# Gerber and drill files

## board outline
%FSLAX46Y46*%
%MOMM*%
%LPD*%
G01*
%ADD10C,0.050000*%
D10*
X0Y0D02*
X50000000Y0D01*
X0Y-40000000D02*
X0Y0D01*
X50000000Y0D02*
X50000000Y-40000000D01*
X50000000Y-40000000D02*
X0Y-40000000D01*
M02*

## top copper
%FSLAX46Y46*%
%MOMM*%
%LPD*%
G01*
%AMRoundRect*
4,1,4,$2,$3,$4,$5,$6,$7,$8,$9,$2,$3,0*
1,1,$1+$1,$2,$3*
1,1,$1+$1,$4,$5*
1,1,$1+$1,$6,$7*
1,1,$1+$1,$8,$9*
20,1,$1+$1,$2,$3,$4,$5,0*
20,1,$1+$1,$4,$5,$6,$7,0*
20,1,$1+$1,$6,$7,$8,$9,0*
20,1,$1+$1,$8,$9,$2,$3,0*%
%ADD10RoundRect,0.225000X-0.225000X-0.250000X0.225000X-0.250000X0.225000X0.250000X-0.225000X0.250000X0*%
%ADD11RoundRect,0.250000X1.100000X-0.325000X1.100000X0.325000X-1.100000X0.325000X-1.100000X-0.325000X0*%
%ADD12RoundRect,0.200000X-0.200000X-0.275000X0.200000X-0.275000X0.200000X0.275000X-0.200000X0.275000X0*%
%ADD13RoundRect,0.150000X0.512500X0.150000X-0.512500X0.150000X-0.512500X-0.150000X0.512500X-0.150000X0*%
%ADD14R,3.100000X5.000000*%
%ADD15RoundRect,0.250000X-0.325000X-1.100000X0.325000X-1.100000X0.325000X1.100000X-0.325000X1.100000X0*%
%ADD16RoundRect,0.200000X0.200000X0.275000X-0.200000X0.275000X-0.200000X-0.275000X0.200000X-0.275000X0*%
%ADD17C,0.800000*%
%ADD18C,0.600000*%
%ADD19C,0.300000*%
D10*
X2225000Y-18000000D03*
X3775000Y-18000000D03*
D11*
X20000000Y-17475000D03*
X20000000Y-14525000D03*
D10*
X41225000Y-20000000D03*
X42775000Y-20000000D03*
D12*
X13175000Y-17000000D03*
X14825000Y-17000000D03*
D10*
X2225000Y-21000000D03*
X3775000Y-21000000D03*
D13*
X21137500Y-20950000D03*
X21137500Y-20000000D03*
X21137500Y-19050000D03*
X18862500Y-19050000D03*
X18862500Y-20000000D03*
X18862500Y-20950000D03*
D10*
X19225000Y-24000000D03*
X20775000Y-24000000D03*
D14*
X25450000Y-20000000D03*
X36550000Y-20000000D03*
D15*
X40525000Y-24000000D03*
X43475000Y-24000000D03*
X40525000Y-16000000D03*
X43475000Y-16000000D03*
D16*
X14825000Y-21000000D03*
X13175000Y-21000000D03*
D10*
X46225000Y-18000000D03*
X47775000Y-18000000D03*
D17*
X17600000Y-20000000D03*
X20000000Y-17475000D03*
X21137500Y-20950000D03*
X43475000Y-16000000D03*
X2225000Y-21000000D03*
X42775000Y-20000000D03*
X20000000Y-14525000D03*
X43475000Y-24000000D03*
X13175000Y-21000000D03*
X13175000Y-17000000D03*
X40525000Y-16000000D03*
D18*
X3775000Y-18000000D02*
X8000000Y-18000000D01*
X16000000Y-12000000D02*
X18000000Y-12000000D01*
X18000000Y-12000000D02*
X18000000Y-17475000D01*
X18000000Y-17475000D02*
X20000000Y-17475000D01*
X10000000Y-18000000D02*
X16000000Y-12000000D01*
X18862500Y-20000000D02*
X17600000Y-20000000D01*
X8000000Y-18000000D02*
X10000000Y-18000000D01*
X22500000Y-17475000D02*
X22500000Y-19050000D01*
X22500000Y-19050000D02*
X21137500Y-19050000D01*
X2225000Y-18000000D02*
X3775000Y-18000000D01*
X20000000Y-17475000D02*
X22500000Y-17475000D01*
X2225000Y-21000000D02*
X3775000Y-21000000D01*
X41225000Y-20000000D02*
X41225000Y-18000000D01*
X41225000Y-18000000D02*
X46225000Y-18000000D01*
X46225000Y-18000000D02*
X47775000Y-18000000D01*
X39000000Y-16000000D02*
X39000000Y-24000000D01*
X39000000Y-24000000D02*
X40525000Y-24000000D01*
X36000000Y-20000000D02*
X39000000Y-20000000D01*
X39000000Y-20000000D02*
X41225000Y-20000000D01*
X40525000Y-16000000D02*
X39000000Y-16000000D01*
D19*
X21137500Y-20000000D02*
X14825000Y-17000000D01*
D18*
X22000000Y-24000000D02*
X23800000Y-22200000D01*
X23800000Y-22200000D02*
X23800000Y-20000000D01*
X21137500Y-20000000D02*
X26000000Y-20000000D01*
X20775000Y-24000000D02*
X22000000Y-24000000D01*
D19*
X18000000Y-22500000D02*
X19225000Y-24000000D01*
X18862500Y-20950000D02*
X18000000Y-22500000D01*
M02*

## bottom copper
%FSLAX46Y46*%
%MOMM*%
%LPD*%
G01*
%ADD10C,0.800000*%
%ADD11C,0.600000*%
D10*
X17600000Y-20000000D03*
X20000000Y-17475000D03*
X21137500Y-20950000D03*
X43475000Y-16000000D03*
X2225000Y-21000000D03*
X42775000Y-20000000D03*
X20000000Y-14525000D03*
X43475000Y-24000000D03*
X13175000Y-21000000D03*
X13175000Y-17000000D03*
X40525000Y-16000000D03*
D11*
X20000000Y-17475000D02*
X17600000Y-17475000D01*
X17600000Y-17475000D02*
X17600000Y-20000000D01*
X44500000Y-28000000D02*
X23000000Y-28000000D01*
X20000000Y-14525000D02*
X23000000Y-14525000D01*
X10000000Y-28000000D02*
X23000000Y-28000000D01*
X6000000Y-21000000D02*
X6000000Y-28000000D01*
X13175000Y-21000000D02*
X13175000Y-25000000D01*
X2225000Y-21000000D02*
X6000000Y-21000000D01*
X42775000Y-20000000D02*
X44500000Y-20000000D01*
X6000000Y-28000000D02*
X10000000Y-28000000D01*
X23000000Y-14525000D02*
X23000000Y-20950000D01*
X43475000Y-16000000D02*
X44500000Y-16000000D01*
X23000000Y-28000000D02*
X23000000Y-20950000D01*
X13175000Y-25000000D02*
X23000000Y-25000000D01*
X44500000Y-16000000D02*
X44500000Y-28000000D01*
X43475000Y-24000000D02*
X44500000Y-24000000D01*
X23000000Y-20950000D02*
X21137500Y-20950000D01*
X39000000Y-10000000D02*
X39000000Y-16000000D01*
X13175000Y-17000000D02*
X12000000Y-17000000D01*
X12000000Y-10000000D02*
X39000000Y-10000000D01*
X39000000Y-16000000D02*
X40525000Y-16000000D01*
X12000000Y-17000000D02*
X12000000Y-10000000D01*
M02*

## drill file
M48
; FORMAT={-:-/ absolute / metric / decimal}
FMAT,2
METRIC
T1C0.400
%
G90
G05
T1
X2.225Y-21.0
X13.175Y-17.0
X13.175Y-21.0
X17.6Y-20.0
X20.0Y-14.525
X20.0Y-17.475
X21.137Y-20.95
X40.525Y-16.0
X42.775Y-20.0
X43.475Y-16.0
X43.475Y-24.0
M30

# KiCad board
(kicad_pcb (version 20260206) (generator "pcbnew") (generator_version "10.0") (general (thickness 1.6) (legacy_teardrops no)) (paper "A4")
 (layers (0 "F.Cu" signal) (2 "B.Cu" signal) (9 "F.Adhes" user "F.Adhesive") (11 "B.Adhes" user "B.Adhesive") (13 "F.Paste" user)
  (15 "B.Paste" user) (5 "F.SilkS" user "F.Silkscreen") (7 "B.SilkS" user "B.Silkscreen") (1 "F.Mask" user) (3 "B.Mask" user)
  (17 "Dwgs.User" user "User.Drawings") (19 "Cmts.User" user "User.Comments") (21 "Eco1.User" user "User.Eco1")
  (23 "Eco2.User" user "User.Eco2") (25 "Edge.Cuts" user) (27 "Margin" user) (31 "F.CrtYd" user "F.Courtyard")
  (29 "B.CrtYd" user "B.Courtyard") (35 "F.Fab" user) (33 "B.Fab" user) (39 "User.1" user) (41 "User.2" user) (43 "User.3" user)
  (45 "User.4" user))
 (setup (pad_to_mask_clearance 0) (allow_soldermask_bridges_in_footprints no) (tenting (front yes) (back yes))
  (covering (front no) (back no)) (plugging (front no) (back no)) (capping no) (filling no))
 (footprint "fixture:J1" (layer "F.Cu") (at 3 18)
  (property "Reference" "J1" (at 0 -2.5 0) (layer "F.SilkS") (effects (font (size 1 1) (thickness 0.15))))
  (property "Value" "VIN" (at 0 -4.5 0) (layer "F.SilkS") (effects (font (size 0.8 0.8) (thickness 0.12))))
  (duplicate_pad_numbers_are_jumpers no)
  (pad "1" smd roundrect (at -0.775 0) (size 0.9 0.95) (layers "F.Cu" "F.Mask" "F.Paste") (roundrect_rratio 0.25) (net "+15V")
   (thermal_bridge_angle 45))
  (pad "2" smd roundrect (at 0.775 0) (size 0.9 0.95) (layers "F.Cu" "F.Mask" "F.Paste") (roundrect_rratio 0.25) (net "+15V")
   (thermal_bridge_angle 45)))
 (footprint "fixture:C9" (layer "F.Cu") (at 20 16 90)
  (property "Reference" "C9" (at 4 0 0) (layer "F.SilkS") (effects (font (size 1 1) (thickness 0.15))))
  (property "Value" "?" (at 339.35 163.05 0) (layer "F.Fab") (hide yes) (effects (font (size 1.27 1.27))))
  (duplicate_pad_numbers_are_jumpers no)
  (pad "1" smd roundrect (at -1.475 0 90) (size 1.15 2.7) (layers "F.Cu" "F.Mask" "F.Paste") (roundrect_rratio 0.217391) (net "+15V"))
  (pad "2" smd roundrect (at 1.475 0 90) (size 1.15 2.7) (layers "F.Cu" "F.Mask" "F.Paste") (roundrect_rratio 0.217391) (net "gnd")))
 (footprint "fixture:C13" (layer "F.Cu") (at 42 20)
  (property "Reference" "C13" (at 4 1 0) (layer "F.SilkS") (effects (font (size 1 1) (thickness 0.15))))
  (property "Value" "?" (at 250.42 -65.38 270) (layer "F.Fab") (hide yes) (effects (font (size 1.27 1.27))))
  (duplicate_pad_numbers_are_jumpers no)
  (pad "1" smd roundrect (at -0.775 0) (size 0.9 0.95) (layers "F.Cu" "F.Mask" "F.Paste") (roundrect_rratio 0.25) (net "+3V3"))
  (pad "2" smd roundrect (at 0.775 0) (size 0.9 0.95) (layers "F.Cu" "F.Mask" "F.Paste") (roundrect_rratio 0.25) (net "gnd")))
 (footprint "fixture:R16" (layer "F.Cu") (at 14 17)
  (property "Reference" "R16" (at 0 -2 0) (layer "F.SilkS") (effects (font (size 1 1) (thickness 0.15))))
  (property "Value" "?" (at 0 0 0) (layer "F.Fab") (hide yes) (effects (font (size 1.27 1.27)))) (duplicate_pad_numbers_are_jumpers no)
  (pad "1" smd roundrect (at -0.825 0) (size 0.8 0.95) (layers "F.Cu" "F.Mask" "F.Paste") (roundrect_rratio 0.25) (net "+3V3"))
  (pad "2" smd roundrect (at 0.825 0) (size 0.8 0.95) (layers "F.Cu" "F.Mask" "F.Paste") (roundrect_rratio 0.25) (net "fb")))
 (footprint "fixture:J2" (layer "F.Cu") (at 3 21)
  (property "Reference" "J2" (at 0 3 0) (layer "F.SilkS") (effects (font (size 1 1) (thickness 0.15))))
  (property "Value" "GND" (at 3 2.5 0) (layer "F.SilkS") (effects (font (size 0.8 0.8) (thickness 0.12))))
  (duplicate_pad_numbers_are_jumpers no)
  (pad "1" smd roundrect (at -0.775 0) (size 0.9 0.95) (layers "F.Cu" "F.Mask" "F.Paste") (roundrect_rratio 0.25) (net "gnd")
   (thermal_bridge_angle 45))
  (pad "2" smd roundrect (at 0.775 0) (size 0.9 0.95) (layers "F.Cu" "F.Mask" "F.Paste") (roundrect_rratio 0.25) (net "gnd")
   (thermal_bridge_angle 45)))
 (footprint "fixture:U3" (layer "F.Cu") (at 20 20 180)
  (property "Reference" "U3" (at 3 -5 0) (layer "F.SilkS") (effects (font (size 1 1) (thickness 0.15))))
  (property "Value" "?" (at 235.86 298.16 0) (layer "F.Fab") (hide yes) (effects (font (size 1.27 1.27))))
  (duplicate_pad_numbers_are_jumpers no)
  (pad "1" smd roundrect (at -1.1375 -0.95 180) (size 1.325 0.6) (layers "F.Cu" "F.Mask" "F.Paste") (roundrect_rratio 0.25) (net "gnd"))
  (pad "2" smd roundrect (at -1.1375 0 180) (size 1.325 0.6) (layers "F.Cu" "F.Mask" "F.Paste") (roundrect_rratio 0.25) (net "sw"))
  (pad "3" smd roundrect (at -1.1375 0.95 180) (size 1.325 0.6) (layers "F.Cu" "F.Mask" "F.Paste") (roundrect_rratio 0.25) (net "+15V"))
  (pad "4" smd roundrect (at 1.1375 0.95 180) (size 1.325 0.6) (layers "F.Cu" "F.Mask" "F.Paste") (roundrect_rratio 0.25) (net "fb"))
  (pad "5" smd roundrect (at 1.1375 0 180) (size 1.325 0.6) (layers "F.Cu" "F.Mask" "F.Paste") (roundrect_rratio 0.25) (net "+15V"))
  (pad "6" smd roundrect (at 1.1375 -0.95 180) (size 1.325 0.6) (layers "F.Cu" "F.Mask" "F.Paste") (roundrect_rratio 0.25) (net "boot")))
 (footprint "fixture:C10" (layer "F.Cu") (at 20 24)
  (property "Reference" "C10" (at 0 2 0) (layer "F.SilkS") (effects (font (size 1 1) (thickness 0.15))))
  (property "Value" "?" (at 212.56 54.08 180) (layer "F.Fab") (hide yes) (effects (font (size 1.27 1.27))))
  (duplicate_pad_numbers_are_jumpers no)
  (pad "1" smd roundrect (at -0.775 0) (size 0.9 0.95) (layers "F.Cu" "F.Mask" "F.Paste") (roundrect_rratio 0.25) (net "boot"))
  (pad "2" smd roundrect (at 0.775 0) (size 0.9 0.95) (layers "F.Cu" "F.Mask" "F.Paste") (roundrect_rratio 0.25) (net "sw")))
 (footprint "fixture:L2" (layer "F.Cu") (at 31 20)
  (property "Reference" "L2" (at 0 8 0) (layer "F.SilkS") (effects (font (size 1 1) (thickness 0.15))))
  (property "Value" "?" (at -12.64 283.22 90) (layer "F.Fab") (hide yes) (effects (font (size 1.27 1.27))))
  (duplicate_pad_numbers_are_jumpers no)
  (pad "1" smd rect (at -5.55 0) (size 3.1 5) (layers "F.Cu" "F.Mask" "F.Paste") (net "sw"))
  (pad "2" smd rect (at 5.55 0) (size 3.1 5) (layers "F.Cu" "F.Mask" "F.Paste") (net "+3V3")))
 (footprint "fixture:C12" (layer "F.Cu") (at 42 24)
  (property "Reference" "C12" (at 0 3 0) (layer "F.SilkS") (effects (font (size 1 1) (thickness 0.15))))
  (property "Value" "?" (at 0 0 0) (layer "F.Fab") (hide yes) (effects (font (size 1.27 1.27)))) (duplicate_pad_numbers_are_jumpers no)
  (pad "1" smd roundrect (at -1.475 0) (size 1.15 2.7) (layers "F.Cu" "F.Mask" "F.Paste") (roundrect_rratio 0.217391) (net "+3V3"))
  (pad "2" smd roundrect (at 1.475 0) (size 1.15 2.7) (layers "F.Cu" "F.Mask" "F.Paste") (roundrect_rratio 0.217391) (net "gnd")))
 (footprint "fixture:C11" (layer "F.Cu") (at 42 16)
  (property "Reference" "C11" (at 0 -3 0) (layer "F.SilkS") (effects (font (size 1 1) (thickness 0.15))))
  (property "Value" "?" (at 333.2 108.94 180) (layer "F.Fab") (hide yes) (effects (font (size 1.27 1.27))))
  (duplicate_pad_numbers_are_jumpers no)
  (pad "1" smd roundrect (at -1.475 0) (size 1.15 2.7) (layers "F.Cu" "F.Mask" "F.Paste") (roundrect_rratio 0.217391) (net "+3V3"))
  (pad "2" smd roundrect (at 1.475 0) (size 1.15 2.7) (layers "F.Cu" "F.Mask" "F.Paste") (roundrect_rratio 0.217391) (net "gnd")))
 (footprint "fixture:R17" (layer "F.Cu") (at 14 21 180)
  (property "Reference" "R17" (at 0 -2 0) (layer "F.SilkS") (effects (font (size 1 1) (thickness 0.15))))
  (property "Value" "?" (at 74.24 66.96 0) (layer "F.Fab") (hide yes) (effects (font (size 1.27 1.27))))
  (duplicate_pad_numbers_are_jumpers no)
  (pad "1" smd roundrect (at -0.825 0 180) (size 0.8 0.95) (layers "F.Cu" "F.Mask" "F.Paste") (roundrect_rratio 0.25) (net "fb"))
  (pad "2" smd roundrect (at 0.825 0 180) (size 0.8 0.95) (layers "F.Cu" "F.Mask" "F.Paste") (roundrect_rratio 0.25) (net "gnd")))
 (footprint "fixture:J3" (layer "F.Cu") (at 47 18)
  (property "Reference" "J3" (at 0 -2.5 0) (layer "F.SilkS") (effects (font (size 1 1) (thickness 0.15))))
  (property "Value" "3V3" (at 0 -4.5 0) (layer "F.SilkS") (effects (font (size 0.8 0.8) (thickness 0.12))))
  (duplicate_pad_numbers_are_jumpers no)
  (pad "1" smd roundrect (at -0.775 0) (size 0.9 0.95) (layers "F.Cu" "F.Mask" "F.Paste") (roundrect_rratio 0.25) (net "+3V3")
   (thermal_bridge_angle 45))
  (pad "2" smd roundrect (at 0.775 0) (size 0.9 0.95) (layers "F.Cu" "F.Mask" "F.Paste") (roundrect_rratio 0.25) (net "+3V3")
   (thermal_bridge_angle 45)))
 (gr_line (start 0 0) (end 50 0) (stroke (width 0.05) (type default)) (layer "Edge.Cuts"))
 (gr_line (start 0 40) (end 0 0) (stroke (width 0.05) (type default)) (layer "Edge.Cuts"))
 (gr_line (start 50 0) (end 50 40) (stroke (width 0.05) (type default)) (layer "Edge.Cuts"))
 (gr_line (start 50 40) (end 0 40) (stroke (width 0.05) (type default)) (layer "Edge.Cuts"))
 (segment (start 3.775 18) (end 8 18) (width 0.6) (layer "F.Cu") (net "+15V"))
 (segment (start 16 12) (end 18 12) (width 0.6) (layer "F.Cu") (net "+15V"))
 (segment (start 18 12) (end 18 17.475) (width 0.6) (layer "F.Cu") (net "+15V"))
 (segment (start 18 17.475) (end 20 17.475) (width 0.6) (layer "F.Cu") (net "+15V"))
 (segment (start 10 18) (end 16 12) (width 0.6) (layer "F.Cu") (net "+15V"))
 (segment (start 18.8625 20) (end 17.6 20) (width 0.6) (layer "F.Cu") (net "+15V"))
 (segment (start 8 18) (end 10 18) (width 0.6) (layer "F.Cu") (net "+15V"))
 (segment (start 22.5 17.475) (end 22.5 19.05) (width 0.6) (layer "F.Cu") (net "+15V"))
 (segment (start 22.5 19.05) (end 21.1375 19.05) (width 0.6) (layer "F.Cu") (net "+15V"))
 (segment (start 2.225 18) (end 3.775 18) (width 0.6) (layer "F.Cu") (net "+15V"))
 (segment (start 20 17.475) (end 22.5 17.475) (width 0.6) (layer "F.Cu") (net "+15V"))
 (via (at 17.6 20) (size 0.8) (drill 0.4) (layers "F.Cu" "B.Cu") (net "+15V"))
 (via (at 20 17.475) (size 0.8) (drill 0.4) (layers "F.Cu" "B.Cu") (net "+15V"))
 (segment (start 20 17.475) (end 17.6 17.475) (width 0.6) (layer "B.Cu") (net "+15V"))
 (segment (start 17.6 17.475) (end 17.6 20) (width 0.6) (layer "B.Cu") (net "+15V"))
 (segment (start 2.225 21) (end 3.775 21) (width 0.6) (layer "F.Cu") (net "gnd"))
 (via (at 21.1375 20.95) (size 0.8) (drill 0.4) (layers "F.Cu" "B.Cu") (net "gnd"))
 (via (at 43.475 16) (size 0.8) (drill 0.4) (layers "F.Cu" "B.Cu") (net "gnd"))
 (via (at 2.225 21) (size 0.8) (drill 0.4) (layers "F.Cu" "B.Cu") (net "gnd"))
 (via (at 42.775 20) (size 0.8) (drill 0.4) (layers "F.Cu" "B.Cu") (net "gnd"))
 (via (at 20 14.525) (size 0.8) (drill 0.4) (layers "F.Cu" "B.Cu") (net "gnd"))
 (via (at 43.475 24) (size 0.8) (drill 0.4) (layers "F.Cu" "B.Cu") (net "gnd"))
 (via (at 13.175 21) (size 0.8) (drill 0.4) (layers "F.Cu" "B.Cu") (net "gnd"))
 (segment (start 44.5 28) (end 23 28) (width 0.6) (layer "B.Cu") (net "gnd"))
 (segment (start 20 14.525) (end 23 14.525) (width 0.6) (layer "B.Cu") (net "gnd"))
 (segment (start 10 28) (end 23 28) (width 0.6) (layer "B.Cu") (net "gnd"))
 (segment (start 6 21) (end 6 28) (width 0.6) (layer "B.Cu") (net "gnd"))
 (segment (start 13.175 21) (end 13.175 25) (width 0.6) (layer "B.Cu") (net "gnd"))
 (segment (start 2.225 21) (end 6 21) (width 0.6) (layer "B.Cu") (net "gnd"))
 (segment (start 42.775 20) (end 44.5 20) (width 0.6) (layer "B.Cu") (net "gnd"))
 (segment (start 6 28) (end 10 28) (width 0.6) (layer "B.Cu") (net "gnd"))
 (segment (start 23 14.525) (end 23 20.95) (width 0.6) (layer "B.Cu") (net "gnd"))
 (segment (start 43.475 16) (end 44.5 16) (width 0.6) (layer "B.Cu") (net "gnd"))
 (segment (start 23 28) (end 23 20.95) (width 0.6) (layer "B.Cu") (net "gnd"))
 (segment (start 13.175 25) (end 23 25) (width 0.6) (layer "B.Cu") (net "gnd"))
 (segment (start 44.5 16) (end 44.5 28) (width 0.6) (layer "B.Cu") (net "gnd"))
 (segment (start 43.475 24) (end 44.5 24) (width 0.6) (layer "B.Cu") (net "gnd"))
 (segment (start 23 20.95) (end 21.1375 20.95) (width 0.6) (layer "B.Cu") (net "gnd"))
 (segment (start 41.225 20) (end 41.225 18) (width 0.6) (layer "F.Cu") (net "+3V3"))
 (segment (start 41.225 18) (end 46.225 18) (width 0.6) (layer "F.Cu") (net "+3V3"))
 (segment (start 46.225 18) (end 47.775 18) (width 0.6) (layer "F.Cu") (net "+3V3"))
 (segment (start 39 16) (end 39 24) (width 0.6) (layer "F.Cu") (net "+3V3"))
 (segment (start 39 24) (end 40.525 24) (width 0.6) (layer "F.Cu") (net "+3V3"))
 (segment (start 36 20) (end 39 20) (width 0.6) (layer "F.Cu") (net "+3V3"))
 (segment (start 39 20) (end 41.225 20) (width 0.6) (layer "F.Cu") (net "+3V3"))
 (segment (start 40.525 16) (end 39 16) (width 0.6) (layer "F.Cu") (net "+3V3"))
 (via (at 13.175 17) (size 0.8) (drill 0.4) (layers "F.Cu" "B.Cu") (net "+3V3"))
 (via (at 40.525 16) (size 0.8) (drill 0.4) (layers "F.Cu" "B.Cu") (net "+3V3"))
 (segment (start 39 10) (end 39 16) (width 0.6) (layer "B.Cu") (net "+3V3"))
 (segment (start 13.175 17) (end 12 17) (width 0.6) (layer "B.Cu") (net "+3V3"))
 (segment (start 12 10) (end 39 10) (width 0.6) (layer "B.Cu") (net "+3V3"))
 (segment (start 39 16) (end 40.525 16) (width 0.6) (layer "B.Cu") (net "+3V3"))
 (segment (start 12 17) (end 12 10) (width 0.6) (layer "B.Cu") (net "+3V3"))
 (segment (start 21.1375 20) (end 14.825 17) (width 0.3) (layer "F.Cu") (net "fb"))
 (segment (start 22 24) (end 23.8 22.2) (width 0.6) (layer "F.Cu") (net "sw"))
 (segment (start 23.8 22.2) (end 23.8 20) (width 0.6) (layer "F.Cu") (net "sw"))
 (segment (start 21.1375 20) (end 26 20) (width 0.6) (layer "F.Cu") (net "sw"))
 (segment (start 20.775 24) (end 22 24) (width 0.6) (layer "F.Cu") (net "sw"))
 (segment (start 18 22.5) (end 19.225 24) (width 0.3) (layer "F.Cu") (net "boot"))
 (segment (start 18.8625 20.95) (end 18 22.5) (width 0.3) (layer "F.Cu") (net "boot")))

